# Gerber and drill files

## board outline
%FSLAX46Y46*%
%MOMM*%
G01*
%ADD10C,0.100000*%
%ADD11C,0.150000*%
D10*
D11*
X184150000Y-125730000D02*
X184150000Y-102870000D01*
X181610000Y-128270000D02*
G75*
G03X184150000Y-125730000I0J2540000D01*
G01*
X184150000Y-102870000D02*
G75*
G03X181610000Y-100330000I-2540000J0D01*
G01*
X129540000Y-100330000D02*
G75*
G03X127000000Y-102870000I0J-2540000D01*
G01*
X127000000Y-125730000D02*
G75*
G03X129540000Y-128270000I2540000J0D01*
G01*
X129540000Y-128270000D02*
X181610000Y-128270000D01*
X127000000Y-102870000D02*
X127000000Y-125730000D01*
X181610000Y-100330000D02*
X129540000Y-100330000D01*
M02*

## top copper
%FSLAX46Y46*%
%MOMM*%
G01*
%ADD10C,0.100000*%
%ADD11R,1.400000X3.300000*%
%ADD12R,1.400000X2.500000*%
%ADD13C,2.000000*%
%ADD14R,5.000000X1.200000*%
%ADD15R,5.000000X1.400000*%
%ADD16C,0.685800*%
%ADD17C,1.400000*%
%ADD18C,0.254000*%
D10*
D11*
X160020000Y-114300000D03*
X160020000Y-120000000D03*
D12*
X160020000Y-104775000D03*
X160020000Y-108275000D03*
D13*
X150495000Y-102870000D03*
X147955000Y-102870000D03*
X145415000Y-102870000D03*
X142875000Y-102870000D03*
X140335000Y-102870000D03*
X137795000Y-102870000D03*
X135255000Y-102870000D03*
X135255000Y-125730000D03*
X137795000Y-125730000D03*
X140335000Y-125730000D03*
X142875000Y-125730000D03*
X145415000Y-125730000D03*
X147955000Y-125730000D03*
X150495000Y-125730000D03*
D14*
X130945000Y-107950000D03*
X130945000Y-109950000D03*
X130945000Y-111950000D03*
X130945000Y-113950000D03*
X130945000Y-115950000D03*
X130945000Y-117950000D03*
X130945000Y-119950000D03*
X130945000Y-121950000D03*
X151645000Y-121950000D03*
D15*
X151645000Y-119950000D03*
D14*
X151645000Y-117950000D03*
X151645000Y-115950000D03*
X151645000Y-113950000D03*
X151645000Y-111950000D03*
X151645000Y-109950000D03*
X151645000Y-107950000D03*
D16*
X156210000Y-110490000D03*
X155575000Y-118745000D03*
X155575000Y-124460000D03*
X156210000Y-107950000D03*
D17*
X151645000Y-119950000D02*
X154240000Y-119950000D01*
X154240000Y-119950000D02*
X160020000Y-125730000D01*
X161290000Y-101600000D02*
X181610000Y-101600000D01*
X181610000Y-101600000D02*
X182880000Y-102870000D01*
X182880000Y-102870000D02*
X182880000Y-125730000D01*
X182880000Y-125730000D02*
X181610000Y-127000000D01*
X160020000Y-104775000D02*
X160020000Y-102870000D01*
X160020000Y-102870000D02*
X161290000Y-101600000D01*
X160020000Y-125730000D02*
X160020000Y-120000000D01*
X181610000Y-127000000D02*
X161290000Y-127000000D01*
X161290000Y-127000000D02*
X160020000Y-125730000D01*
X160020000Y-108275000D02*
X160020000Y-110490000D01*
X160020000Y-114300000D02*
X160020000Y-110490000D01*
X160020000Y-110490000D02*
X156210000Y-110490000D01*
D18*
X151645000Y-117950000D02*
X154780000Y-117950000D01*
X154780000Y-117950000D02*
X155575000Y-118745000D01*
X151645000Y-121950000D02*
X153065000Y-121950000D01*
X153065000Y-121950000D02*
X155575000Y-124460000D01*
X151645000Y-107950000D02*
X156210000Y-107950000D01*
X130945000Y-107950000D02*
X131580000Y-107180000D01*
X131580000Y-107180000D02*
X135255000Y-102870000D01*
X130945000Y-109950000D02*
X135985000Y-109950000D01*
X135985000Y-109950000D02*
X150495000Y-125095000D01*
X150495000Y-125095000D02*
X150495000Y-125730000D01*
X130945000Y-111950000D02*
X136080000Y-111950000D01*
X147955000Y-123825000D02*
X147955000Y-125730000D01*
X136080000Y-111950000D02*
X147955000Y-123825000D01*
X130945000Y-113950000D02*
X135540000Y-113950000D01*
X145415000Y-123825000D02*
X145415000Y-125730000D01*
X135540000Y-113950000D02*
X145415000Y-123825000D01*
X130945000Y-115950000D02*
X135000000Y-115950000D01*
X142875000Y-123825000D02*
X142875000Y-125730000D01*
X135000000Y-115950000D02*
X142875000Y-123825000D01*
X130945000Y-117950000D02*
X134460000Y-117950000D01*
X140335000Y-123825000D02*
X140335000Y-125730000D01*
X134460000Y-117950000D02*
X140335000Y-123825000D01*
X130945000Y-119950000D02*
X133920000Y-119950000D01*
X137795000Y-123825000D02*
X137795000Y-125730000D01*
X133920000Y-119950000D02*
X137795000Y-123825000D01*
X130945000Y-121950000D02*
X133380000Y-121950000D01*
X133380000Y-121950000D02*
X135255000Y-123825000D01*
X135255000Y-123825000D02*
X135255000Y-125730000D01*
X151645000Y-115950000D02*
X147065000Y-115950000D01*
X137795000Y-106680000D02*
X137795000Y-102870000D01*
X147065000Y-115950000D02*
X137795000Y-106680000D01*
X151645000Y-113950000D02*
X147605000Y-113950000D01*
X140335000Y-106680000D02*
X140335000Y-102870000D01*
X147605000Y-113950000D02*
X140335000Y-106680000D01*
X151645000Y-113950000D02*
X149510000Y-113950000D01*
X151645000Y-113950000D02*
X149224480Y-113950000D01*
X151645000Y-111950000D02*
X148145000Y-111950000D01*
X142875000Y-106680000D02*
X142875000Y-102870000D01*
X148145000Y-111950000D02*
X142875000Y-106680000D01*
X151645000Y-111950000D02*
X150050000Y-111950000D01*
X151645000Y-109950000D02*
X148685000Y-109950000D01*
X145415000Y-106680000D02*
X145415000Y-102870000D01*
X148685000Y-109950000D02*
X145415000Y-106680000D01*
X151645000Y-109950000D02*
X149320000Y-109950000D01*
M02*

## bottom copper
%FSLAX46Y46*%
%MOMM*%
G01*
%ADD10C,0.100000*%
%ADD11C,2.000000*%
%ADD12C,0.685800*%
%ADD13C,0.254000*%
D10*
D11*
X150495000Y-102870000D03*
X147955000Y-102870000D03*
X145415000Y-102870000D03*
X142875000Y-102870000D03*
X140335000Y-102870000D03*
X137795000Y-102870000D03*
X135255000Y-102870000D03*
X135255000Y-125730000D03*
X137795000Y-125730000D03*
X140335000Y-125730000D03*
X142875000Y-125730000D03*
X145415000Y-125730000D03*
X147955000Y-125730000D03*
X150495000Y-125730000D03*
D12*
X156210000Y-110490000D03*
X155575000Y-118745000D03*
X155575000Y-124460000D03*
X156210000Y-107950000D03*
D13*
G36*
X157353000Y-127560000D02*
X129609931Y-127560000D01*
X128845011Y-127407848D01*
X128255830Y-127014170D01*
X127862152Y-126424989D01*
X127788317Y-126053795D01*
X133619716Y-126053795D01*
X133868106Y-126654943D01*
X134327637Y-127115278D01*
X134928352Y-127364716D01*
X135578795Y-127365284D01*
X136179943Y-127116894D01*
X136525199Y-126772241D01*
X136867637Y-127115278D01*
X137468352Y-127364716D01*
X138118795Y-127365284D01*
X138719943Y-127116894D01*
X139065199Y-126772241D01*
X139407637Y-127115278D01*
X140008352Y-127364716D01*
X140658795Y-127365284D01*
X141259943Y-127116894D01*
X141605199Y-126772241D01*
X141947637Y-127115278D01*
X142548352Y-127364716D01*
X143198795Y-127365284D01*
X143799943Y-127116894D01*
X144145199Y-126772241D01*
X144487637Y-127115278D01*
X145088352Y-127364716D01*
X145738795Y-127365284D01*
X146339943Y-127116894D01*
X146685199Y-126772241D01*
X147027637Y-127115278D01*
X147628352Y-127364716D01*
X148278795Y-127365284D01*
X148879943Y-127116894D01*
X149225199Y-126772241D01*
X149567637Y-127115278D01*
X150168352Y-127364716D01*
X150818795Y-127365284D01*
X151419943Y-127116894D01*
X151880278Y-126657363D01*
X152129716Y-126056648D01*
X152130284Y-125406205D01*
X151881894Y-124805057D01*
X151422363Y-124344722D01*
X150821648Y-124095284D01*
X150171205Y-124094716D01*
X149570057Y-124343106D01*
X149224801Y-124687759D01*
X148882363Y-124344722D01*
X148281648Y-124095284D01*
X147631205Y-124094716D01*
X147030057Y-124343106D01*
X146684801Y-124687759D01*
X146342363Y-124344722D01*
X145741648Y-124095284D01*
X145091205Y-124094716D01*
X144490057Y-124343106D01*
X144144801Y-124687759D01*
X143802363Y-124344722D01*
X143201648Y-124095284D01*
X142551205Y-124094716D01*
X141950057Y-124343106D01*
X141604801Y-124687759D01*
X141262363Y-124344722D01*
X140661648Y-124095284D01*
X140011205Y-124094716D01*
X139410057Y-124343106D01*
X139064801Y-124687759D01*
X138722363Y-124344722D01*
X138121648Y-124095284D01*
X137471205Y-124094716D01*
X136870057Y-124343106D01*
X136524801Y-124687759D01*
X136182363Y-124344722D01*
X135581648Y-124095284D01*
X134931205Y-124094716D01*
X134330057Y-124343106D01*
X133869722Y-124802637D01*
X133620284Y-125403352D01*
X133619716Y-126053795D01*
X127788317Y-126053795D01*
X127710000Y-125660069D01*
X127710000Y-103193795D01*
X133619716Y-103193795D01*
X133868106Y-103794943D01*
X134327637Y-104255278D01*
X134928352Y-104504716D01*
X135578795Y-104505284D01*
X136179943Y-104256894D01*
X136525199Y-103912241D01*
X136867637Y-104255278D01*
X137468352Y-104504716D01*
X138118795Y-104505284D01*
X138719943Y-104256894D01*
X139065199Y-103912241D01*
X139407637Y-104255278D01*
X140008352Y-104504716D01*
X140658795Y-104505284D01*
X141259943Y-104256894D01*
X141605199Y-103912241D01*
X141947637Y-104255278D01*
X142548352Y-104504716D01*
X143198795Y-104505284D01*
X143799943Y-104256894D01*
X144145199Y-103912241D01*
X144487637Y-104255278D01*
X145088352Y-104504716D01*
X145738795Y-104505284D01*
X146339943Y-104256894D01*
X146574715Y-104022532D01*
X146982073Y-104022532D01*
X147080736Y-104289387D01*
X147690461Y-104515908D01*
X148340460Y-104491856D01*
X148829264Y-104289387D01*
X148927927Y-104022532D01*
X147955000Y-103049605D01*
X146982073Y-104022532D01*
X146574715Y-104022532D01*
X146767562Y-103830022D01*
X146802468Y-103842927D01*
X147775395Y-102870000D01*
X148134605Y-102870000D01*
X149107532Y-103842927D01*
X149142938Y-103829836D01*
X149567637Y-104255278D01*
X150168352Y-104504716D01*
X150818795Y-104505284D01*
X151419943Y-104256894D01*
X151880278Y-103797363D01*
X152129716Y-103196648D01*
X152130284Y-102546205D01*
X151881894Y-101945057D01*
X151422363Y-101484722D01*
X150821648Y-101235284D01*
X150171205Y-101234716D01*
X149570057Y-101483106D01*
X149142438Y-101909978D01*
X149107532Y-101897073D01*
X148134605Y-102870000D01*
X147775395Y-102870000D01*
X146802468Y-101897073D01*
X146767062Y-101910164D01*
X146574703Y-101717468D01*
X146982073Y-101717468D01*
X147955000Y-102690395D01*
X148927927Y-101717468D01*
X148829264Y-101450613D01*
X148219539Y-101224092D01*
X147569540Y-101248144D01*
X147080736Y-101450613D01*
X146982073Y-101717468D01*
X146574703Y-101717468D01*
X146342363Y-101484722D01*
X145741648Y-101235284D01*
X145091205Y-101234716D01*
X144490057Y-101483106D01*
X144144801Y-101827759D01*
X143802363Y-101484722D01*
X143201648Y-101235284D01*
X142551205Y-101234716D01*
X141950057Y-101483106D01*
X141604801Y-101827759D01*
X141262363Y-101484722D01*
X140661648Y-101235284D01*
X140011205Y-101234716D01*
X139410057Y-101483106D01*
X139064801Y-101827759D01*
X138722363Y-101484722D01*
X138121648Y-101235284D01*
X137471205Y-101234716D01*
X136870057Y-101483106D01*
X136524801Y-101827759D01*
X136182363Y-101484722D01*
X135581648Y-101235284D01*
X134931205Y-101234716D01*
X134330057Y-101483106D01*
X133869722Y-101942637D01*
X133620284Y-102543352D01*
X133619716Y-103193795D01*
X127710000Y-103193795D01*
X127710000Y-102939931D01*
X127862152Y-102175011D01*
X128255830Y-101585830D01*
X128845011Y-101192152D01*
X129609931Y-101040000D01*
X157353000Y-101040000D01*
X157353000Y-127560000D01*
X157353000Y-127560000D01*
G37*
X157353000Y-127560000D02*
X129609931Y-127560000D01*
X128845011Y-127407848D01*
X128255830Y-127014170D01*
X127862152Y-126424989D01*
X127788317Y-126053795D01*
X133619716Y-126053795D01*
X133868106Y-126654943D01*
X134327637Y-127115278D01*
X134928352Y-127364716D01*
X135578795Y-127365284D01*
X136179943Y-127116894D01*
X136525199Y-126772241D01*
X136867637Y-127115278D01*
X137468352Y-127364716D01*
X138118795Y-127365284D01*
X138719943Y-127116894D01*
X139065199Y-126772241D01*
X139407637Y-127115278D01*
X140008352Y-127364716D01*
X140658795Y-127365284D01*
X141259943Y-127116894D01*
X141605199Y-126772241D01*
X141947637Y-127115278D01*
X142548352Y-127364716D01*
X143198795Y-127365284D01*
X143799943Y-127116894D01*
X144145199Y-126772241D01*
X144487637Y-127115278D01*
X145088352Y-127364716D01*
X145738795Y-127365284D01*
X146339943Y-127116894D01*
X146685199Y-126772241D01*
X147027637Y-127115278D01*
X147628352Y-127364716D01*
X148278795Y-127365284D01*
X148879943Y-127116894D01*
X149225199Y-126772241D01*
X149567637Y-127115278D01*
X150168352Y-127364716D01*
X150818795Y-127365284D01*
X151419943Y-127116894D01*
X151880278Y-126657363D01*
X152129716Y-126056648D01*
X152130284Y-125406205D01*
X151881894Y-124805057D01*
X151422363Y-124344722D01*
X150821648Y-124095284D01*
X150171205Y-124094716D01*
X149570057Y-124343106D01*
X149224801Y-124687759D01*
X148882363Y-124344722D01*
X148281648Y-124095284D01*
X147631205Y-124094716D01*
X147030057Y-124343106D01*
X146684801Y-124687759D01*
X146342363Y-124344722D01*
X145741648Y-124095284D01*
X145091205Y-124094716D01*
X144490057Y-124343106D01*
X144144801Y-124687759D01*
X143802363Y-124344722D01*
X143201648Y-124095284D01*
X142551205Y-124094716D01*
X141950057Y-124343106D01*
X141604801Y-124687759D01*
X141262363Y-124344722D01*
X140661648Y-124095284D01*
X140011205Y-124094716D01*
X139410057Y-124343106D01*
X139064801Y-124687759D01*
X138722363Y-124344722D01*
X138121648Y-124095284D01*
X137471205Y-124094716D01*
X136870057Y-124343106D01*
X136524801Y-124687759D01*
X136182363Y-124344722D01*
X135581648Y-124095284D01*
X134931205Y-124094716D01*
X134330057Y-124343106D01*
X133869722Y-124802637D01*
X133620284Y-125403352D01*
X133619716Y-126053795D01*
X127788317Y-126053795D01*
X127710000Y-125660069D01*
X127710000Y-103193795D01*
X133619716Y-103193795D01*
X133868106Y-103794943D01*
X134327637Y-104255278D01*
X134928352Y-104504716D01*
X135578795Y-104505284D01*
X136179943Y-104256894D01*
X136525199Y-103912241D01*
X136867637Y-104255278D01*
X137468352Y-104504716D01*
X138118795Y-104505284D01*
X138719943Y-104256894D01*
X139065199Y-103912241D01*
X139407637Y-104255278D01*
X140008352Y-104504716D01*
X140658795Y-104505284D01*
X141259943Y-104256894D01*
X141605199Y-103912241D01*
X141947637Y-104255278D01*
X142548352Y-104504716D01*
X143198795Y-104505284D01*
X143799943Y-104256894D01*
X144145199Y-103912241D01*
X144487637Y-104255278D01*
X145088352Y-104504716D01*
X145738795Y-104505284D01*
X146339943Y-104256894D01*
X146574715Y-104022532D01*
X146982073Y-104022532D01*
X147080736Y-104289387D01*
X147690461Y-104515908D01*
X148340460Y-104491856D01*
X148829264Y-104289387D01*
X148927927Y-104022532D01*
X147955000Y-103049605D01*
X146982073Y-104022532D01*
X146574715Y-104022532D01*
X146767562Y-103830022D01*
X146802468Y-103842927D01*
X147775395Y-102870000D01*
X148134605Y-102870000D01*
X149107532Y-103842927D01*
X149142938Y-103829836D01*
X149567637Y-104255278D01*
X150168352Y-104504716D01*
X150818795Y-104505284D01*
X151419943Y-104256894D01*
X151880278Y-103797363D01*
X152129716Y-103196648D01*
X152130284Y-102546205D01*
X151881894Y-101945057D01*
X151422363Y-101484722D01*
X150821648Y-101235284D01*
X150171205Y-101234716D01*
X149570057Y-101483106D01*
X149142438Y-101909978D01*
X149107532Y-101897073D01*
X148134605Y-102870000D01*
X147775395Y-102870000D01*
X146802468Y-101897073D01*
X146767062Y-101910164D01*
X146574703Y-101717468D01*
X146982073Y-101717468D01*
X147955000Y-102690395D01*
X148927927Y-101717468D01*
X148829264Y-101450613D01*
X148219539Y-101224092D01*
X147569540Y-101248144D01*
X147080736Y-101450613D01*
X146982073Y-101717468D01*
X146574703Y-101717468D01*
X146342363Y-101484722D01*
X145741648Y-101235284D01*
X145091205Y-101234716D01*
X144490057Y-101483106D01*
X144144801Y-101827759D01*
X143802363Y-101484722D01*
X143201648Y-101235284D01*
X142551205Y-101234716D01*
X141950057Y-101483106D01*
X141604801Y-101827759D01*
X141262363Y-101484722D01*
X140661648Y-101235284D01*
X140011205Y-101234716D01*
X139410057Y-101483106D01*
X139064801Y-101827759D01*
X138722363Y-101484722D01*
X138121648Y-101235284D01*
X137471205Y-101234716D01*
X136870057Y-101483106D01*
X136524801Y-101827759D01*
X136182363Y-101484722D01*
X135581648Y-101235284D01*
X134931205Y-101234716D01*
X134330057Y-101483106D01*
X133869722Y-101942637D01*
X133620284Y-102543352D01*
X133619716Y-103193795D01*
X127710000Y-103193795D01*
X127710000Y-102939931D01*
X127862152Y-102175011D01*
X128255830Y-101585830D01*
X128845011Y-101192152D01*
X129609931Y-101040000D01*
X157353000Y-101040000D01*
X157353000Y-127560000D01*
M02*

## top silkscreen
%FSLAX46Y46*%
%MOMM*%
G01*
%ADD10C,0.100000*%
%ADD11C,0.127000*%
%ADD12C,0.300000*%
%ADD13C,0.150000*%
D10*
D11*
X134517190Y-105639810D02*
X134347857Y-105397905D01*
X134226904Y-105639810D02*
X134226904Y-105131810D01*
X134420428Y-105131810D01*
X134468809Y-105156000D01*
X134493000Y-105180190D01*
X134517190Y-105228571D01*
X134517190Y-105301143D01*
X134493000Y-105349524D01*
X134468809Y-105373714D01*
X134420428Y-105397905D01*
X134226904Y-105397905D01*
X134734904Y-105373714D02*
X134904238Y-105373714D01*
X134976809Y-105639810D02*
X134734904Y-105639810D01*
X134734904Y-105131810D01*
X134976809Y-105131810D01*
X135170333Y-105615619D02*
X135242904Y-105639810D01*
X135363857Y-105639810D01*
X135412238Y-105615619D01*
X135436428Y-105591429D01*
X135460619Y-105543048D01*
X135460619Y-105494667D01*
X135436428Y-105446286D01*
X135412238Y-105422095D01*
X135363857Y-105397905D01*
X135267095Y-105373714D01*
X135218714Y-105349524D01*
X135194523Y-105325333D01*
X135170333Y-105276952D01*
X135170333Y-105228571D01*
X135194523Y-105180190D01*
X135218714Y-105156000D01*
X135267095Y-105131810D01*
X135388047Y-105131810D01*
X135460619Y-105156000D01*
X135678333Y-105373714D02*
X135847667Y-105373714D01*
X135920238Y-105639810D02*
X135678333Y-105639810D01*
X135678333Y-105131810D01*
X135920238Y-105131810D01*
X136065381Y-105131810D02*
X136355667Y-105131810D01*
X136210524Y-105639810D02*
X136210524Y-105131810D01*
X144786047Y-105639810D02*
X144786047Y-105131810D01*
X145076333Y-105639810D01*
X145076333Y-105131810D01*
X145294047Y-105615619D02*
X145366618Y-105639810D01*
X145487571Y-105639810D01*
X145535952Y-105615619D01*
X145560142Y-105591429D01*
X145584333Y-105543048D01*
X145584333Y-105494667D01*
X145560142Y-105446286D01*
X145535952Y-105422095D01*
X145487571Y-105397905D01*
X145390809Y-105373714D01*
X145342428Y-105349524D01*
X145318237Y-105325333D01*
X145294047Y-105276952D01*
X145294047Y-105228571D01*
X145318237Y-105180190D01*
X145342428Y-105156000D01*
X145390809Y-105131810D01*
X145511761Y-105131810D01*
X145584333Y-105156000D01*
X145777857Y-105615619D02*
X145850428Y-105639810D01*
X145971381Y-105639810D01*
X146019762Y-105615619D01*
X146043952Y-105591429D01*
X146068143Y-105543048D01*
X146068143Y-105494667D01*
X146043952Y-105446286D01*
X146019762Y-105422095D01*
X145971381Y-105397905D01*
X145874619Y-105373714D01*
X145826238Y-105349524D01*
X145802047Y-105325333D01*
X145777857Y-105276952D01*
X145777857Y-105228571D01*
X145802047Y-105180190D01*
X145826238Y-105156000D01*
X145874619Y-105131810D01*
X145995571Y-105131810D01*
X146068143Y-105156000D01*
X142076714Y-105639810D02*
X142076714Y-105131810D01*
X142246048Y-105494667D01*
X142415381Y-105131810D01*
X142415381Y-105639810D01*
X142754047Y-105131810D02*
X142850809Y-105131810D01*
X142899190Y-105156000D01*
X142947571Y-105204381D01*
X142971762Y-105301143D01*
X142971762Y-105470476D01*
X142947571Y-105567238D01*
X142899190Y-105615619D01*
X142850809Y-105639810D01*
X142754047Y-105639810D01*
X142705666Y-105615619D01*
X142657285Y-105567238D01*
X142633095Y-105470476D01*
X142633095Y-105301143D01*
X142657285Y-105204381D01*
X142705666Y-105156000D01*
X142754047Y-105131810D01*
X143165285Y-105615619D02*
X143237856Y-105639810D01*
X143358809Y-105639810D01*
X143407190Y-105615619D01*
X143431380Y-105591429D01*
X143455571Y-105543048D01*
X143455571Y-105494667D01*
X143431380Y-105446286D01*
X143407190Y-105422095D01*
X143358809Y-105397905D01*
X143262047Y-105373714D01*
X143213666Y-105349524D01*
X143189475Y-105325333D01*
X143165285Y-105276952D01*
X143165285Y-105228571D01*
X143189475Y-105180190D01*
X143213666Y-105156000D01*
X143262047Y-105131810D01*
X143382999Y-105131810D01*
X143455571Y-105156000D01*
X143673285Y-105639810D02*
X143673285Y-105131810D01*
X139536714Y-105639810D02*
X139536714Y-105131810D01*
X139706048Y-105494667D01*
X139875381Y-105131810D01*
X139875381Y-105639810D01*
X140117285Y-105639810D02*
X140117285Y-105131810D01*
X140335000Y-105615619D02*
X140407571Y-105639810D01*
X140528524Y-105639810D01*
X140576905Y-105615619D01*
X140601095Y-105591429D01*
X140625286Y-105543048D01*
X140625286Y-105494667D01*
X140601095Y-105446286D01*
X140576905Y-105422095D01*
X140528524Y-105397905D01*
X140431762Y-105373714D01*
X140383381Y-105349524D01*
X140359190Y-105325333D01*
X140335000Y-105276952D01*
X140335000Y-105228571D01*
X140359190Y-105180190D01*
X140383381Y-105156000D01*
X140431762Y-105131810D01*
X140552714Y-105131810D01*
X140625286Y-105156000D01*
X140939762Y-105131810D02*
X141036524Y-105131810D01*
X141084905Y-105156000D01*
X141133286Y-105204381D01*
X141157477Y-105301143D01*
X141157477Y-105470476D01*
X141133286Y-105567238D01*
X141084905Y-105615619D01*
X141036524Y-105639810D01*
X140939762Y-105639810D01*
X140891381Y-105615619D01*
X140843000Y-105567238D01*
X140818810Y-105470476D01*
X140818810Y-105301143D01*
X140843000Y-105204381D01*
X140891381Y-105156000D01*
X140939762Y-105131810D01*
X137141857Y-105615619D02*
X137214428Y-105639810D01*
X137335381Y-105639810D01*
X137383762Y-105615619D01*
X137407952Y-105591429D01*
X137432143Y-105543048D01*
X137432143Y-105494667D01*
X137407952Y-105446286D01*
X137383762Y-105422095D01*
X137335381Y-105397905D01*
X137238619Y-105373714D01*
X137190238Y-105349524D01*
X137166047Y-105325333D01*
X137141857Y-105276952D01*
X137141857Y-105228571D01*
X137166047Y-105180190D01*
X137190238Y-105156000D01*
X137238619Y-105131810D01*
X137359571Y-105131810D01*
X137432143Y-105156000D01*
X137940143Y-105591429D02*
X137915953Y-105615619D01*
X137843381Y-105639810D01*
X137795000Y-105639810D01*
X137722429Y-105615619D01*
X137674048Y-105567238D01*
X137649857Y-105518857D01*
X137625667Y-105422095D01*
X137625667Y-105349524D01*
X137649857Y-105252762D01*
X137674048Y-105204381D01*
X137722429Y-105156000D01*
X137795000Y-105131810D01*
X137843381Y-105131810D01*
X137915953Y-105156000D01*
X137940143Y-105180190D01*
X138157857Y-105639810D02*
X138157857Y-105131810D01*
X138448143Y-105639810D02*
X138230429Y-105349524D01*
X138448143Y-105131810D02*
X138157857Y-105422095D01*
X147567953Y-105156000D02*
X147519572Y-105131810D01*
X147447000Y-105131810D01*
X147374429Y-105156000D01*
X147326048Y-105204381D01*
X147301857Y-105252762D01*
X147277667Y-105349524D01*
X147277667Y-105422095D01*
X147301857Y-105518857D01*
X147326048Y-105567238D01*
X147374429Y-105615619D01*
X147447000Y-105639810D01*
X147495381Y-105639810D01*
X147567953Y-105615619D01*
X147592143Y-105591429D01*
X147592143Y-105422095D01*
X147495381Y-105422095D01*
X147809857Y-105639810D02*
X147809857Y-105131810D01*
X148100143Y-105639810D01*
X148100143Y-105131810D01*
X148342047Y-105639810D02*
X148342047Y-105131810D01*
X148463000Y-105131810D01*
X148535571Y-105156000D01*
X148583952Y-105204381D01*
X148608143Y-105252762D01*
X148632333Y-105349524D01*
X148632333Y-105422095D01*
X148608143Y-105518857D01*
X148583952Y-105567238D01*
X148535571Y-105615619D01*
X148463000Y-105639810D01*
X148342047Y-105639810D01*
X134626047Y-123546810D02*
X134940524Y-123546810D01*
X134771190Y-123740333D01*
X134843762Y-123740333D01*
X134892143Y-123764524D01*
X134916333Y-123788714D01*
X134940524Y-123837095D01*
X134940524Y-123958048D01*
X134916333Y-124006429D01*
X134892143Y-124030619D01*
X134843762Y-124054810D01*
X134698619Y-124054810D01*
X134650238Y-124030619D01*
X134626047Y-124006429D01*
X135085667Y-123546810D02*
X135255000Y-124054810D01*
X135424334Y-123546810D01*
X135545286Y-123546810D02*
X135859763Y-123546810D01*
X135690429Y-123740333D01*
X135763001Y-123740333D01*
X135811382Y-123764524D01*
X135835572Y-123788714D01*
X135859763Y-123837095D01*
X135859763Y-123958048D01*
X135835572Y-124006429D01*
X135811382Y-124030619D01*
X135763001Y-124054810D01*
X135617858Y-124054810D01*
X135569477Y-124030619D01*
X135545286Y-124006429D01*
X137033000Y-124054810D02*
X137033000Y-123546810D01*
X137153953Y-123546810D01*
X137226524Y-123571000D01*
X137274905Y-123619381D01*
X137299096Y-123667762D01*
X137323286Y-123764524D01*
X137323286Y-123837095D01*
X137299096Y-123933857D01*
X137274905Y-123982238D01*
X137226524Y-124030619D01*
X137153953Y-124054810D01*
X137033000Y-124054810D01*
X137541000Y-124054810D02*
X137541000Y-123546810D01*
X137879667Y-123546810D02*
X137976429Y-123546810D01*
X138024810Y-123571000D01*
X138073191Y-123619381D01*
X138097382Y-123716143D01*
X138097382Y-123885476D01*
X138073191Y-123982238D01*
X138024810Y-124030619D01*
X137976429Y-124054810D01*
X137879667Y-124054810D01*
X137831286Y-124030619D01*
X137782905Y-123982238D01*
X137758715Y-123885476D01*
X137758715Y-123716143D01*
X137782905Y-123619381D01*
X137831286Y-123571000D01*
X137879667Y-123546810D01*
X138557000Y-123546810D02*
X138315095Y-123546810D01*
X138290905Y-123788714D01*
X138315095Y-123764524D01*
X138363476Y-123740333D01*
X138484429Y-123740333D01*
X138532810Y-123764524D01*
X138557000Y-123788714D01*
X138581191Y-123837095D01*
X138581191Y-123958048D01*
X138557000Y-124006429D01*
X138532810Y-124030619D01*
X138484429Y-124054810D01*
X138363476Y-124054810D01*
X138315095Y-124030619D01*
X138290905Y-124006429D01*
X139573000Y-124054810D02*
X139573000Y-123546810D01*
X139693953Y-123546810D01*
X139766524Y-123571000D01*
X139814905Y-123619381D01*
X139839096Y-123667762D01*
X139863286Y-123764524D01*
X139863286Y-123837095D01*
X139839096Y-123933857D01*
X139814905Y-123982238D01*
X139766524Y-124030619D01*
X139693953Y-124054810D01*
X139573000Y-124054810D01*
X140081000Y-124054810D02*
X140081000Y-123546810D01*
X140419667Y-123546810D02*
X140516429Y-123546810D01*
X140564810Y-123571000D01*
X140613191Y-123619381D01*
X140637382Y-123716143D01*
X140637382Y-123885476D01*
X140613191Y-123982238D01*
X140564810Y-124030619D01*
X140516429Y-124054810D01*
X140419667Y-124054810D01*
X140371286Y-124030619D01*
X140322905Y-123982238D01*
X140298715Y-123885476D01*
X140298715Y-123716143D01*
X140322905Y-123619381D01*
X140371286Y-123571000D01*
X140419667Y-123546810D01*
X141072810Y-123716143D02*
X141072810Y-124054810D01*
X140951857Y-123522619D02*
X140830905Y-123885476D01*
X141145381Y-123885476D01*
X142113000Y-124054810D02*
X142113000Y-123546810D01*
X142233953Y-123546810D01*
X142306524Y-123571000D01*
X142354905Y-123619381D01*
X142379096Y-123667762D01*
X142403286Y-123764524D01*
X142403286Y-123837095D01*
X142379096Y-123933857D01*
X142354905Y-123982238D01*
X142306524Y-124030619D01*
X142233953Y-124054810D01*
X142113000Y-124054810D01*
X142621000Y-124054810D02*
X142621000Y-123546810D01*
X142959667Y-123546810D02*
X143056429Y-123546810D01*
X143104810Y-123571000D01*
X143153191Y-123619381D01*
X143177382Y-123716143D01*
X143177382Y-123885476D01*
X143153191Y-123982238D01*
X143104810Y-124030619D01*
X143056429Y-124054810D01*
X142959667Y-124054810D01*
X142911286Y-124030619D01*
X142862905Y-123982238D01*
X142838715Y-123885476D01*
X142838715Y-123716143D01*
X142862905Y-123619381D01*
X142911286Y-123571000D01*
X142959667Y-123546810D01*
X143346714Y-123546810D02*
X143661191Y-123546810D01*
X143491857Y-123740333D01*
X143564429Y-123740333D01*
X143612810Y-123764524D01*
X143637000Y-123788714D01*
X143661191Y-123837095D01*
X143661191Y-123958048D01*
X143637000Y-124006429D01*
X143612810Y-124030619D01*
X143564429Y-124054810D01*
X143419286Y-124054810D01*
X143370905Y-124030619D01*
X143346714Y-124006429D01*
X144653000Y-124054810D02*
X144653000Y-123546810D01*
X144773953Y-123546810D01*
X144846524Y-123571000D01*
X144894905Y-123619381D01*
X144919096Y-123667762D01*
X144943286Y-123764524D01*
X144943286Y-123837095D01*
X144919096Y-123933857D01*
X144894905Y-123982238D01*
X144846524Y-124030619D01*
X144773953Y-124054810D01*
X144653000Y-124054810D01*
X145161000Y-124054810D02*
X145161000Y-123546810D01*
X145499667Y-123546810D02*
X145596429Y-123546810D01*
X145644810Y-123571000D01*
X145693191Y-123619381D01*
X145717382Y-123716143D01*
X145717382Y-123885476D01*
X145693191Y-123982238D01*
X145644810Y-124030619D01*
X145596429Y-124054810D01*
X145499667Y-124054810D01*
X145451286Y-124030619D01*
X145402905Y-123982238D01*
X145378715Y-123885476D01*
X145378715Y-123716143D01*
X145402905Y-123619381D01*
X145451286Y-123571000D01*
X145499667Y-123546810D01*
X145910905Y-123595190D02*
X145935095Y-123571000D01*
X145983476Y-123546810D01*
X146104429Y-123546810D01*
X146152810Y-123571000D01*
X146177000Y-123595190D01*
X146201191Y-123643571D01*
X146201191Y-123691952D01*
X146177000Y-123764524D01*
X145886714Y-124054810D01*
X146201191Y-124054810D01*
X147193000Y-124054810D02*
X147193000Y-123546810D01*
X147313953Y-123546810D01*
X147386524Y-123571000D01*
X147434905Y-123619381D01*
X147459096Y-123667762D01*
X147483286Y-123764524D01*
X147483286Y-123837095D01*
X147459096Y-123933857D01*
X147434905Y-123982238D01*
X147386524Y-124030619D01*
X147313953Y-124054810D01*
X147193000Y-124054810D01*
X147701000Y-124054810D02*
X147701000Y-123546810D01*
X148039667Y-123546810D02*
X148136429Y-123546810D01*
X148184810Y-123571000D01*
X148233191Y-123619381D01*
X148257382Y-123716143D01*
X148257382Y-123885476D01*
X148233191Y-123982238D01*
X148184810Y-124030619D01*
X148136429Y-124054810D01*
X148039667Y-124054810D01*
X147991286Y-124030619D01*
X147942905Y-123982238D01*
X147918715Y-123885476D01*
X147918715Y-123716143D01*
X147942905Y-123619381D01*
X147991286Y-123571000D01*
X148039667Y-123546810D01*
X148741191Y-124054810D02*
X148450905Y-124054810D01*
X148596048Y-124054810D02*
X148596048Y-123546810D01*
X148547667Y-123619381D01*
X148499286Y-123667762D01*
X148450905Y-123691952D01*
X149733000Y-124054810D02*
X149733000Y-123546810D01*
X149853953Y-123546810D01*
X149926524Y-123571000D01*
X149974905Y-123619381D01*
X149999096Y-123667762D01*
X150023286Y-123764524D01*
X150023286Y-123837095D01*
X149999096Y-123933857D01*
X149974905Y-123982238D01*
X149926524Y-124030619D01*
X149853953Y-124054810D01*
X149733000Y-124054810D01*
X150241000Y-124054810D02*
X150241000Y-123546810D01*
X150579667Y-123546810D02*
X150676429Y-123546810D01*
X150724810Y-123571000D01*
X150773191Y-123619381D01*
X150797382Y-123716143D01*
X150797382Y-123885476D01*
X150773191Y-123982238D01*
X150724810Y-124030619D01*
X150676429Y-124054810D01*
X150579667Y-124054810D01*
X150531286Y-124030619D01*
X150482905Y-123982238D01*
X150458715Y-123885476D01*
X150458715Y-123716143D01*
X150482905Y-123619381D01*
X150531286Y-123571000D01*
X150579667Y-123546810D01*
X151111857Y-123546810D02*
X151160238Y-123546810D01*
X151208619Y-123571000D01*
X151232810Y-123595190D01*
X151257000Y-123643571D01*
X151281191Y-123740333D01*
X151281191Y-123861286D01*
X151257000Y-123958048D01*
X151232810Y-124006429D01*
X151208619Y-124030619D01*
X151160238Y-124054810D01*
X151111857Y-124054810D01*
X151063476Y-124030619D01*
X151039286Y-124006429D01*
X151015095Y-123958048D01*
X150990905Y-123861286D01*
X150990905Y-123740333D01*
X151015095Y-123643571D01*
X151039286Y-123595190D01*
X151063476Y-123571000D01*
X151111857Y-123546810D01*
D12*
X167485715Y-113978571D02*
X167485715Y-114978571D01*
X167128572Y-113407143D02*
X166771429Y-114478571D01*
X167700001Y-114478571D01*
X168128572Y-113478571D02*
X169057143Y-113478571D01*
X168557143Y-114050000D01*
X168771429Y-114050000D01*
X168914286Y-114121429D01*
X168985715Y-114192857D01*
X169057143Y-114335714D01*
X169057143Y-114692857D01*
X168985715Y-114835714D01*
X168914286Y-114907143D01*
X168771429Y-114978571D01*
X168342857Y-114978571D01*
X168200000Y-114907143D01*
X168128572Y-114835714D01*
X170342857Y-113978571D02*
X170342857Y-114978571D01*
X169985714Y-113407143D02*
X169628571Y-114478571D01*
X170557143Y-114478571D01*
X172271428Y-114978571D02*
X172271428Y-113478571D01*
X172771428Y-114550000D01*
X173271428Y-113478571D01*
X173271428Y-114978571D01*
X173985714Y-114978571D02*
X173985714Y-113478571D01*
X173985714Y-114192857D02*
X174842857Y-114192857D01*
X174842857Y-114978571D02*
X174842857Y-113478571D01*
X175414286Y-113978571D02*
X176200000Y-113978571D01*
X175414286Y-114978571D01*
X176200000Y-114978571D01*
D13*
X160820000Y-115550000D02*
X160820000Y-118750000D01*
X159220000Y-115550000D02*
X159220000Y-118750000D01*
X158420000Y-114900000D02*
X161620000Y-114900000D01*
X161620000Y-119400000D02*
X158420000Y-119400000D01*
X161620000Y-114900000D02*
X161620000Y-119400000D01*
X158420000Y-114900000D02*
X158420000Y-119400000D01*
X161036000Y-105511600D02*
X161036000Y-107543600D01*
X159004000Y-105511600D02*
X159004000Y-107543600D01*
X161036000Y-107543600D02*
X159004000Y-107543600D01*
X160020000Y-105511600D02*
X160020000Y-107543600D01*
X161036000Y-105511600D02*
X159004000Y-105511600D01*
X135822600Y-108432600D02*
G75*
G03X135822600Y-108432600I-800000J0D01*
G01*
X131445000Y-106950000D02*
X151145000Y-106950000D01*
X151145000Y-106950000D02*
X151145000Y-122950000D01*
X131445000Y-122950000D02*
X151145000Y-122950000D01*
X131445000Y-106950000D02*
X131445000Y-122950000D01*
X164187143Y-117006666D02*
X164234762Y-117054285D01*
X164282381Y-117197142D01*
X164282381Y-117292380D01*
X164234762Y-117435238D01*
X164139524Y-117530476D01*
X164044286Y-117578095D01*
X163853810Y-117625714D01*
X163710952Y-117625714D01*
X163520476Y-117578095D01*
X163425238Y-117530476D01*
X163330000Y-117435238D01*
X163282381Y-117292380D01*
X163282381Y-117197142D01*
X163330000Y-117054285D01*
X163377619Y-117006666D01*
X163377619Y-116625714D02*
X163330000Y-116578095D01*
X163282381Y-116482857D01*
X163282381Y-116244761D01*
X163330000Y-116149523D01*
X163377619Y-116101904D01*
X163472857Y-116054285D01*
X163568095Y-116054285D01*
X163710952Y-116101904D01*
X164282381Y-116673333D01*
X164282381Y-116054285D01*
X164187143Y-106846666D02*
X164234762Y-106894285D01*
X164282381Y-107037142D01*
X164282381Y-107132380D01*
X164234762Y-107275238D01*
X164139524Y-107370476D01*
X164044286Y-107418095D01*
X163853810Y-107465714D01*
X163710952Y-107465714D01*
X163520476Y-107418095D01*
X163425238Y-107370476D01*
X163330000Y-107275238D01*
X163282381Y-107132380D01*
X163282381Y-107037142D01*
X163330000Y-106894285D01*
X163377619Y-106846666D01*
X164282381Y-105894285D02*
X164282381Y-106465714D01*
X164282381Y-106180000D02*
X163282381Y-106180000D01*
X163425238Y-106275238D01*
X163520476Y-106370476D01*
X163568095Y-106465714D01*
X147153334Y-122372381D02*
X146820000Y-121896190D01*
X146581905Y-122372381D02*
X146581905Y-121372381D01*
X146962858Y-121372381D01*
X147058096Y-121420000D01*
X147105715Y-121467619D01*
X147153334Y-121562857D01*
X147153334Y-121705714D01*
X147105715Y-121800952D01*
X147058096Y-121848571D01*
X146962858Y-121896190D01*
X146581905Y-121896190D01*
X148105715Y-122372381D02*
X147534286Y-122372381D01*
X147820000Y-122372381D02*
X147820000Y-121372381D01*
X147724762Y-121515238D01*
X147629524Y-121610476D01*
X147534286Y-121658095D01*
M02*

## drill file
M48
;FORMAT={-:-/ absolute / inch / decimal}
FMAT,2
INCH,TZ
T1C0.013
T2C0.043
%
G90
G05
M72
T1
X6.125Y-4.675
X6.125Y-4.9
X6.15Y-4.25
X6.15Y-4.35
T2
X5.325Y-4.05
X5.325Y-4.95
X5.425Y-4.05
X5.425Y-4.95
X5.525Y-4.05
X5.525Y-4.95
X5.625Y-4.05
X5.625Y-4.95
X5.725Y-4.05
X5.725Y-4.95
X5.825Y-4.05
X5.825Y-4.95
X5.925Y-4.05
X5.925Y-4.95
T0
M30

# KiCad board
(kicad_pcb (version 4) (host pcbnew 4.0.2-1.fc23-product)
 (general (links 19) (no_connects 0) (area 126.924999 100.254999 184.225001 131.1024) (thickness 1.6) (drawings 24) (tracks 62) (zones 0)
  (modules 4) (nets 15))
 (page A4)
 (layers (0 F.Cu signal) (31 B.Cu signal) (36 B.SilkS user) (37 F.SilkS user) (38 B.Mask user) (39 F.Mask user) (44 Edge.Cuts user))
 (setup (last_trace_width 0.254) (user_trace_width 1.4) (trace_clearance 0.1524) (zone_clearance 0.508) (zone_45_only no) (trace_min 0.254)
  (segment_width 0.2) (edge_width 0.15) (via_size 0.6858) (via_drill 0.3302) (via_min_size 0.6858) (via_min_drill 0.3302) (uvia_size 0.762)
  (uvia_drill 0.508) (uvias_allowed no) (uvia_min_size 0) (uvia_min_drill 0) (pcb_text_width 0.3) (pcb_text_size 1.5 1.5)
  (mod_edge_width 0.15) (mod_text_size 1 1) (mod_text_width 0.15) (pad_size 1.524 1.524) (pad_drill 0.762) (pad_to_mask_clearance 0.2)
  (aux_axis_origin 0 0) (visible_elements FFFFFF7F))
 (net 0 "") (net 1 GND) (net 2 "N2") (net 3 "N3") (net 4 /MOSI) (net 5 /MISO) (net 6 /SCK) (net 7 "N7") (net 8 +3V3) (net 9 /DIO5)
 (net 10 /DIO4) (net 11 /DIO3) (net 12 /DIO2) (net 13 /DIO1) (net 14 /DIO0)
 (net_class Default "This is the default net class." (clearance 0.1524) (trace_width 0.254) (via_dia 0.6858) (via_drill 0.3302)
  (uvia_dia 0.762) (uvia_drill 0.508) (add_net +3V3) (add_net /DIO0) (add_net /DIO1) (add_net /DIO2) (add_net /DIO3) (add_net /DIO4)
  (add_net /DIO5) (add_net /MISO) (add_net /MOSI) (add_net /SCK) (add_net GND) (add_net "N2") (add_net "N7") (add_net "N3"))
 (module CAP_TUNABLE (layer F.Cu) (at 160.02 114.3 270)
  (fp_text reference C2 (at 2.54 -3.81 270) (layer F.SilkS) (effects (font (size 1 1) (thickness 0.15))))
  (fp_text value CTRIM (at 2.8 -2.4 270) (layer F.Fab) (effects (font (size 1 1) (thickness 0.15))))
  (fp_line (start 1.25 -0.8) (end 4.45 -0.8) (layer F.SilkS) (width 0.15))
  (fp_line (start 1.25 0.8) (end 4.45 0.8) (layer F.SilkS) (width 0.15))
  (fp_line (start 0.6 1.6) (end 0.6 -1.6) (layer F.SilkS) (width 0.15))
  (fp_line (start 5.1 -1.6) (end 5.1 1.6) (layer F.SilkS) (width 0.15))
  (fp_line (start 0.6 -1.6) (end 5.1 -1.6) (layer F.SilkS) (width 0.15))
  (fp_line (start 0.6 1.6) (end 5.1 1.6) (layer F.SilkS) (width 0.15))
  (pad 1 smd rect (at 0 0 270) (size 3.3 1.4) (layers F.Cu F.Mask) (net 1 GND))
  (pad 2 smd rect (at 5.7 0 270) (size 3.3 1.4) (layers F.Cu F.Mask) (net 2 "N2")))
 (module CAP (layer F.Cu) (at 160.02 104.775 270)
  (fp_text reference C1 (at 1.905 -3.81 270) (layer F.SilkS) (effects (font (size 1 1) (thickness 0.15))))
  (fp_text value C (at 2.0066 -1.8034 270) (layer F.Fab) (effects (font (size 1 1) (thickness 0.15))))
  (fp_line (start 0.7366 -1.016) (end 2.7686 -1.016) (layer F.SilkS) (width 0.15))
  (fp_line (start 0.7366 1.016) (end 2.7686 1.016) (layer F.SilkS) (width 0.15))
  (fp_line (start 2.7686 -1.016) (end 2.7686 1.016) (layer F.SilkS) (width 0.15))
  (fp_line (start 0.7366 0) (end 2.7686 0) (layer F.SilkS) (width 0.15))
  (fp_line (start 0.7366 -1.016) (end 0.7366 1.016) (layer F.SilkS) (width 0.15))
  (pad 1 smd rect (at 0 0 270) (size 2.5 1.4) (layers F.Cu F.Mask) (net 2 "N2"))
  (pad 2 smd rect (at 3.5 0 270) (size 2.5 1.4) (layers F.Cu F.Mask) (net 1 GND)))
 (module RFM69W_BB (layer B.Cu) (at 142.875 115.57 180)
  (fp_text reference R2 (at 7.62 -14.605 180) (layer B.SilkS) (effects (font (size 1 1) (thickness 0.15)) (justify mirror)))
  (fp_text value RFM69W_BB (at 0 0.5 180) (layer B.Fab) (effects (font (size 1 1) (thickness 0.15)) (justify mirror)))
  (pad 14 thru_hole circle (at -7.62 12.7 180) (size 2 2) (drill 1.1) (layers *.Cu *.Mask B.SilkS))
  (pad 8 thru_hole circle (at -5.08 12.7 180) (size 2 2) (drill 1.1) (layers *.Cu *.Mask B.SilkS) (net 1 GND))
  (pad 12 thru_hole circle (at -2.54 12.7 180) (size 2 2) (drill 1.1) (layers *.Cu *.Mask B.SilkS) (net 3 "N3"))
  (pad 11 thru_hole circle (at 0 12.7 180) (size 2 2) (drill 1.1) (layers *.Cu *.Mask B.SilkS) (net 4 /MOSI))
  (pad 10 thru_hole circle (at 2.54 12.7 180) (size 2 2) (drill 1.1) (layers *.Cu *.Mask B.SilkS) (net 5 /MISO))
  (pad 9 thru_hole circle (at 5.08 12.7 180) (size 2 2) (drill 1.1) (layers *.Cu *.Mask B.SilkS) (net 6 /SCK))
  (pad 13 thru_hole circle (at 7.62 12.7 180) (size 2 2) (drill 1.1) (layers *.Cu *.Mask B.SilkS) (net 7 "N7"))
  (pad 7 thru_hole circle (at 7.62 -10.16 180) (size 2 2) (drill 1.1) (layers *.Cu *.Mask B.SilkS) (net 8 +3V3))
  (pad 6 thru_hole circle (at 5.08 -10.16 180) (size 2 2) (drill 1.1) (layers *.Cu *.Mask B.SilkS) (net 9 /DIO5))
  (pad 5 thru_hole circle (at 2.54 -10.16 180) (size 2 2) (drill 1.1) (layers *.Cu *.Mask B.SilkS) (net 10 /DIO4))
  (pad 4 thru_hole circle (at 0 -10.16 180) (size 2 2) (drill 1.1) (layers *.Cu *.Mask B.SilkS) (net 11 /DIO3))
  (pad 3 thru_hole circle (at -2.54 -10.16 180) (size 2 2) (drill 1.1) (layers *.Cu *.Mask B.SilkS) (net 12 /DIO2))
  (pad 2 thru_hole circle (at -5.08 -10.16 180) (size 2 2) (drill 1.1) (layers *.Cu *.Mask B.SilkS) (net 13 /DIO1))
  (pad 1 thru_hole circle (at -7.62 -10.16 180) (size 2 2) (drill 1.1) (layers *.Cu *.Mask B.SilkS) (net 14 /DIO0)))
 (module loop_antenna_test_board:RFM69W (layer F.Cu) (at 131.445 107.95)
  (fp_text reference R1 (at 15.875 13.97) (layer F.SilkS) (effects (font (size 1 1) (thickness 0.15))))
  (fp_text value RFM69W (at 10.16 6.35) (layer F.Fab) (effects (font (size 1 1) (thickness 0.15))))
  (fp_circle (center 3.5776 0.4826) (end 3.5776 1.2826) (layer F.SilkS) (width 0.15))
  (fp_line (start 0 -1) (end 19.7 -1) (layer F.SilkS) (width 0.15))
  (fp_line (start 19.7 -1) (end 19.7 15) (layer F.SilkS) (width 0.15))
  (fp_line (start 0 15) (end 19.7 15) (layer F.SilkS) (width 0.15))
  (fp_line (start 0 -1) (end 0 15) (layer F.SilkS) (width 0.15))
  (pad 1 smd rect (at -0.5 0) (size 5 1.2) (layers F.Cu F.Mask) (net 7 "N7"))
  (pad 2 smd rect (at -0.5 2) (size 5 1.2) (layers F.Cu F.Mask) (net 14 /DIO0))
  (pad 3 smd rect (at -0.5 4) (size 5 1.2) (layers F.Cu F.Mask) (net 13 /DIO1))
  (pad 4 smd rect (at -0.5 6) (size 5 1.2) (layers F.Cu F.Mask) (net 12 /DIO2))
  (pad 5 smd rect (at -0.5 8) (size 5 1.2) (layers F.Cu F.Mask) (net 11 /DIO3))
  (pad 6 smd rect (at -0.5 10) (size 5 1.2) (layers F.Cu F.Mask) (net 10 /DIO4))
  (pad 7 smd rect (at -0.5 12) (size 5 1.2) (layers F.Cu F.Mask) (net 9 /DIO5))
  (pad 8 smd rect (at -0.5 14) (size 5 1.2) (layers F.Cu F.Mask) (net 8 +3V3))
  (pad 9 smd rect (at 20.2 14) (size 5 1.2) (layers F.Cu F.Mask) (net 1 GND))
  (pad 10 smd rect (at 20.2 12) (size 5 1.4) (layers F.Cu F.Mask) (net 2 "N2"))
  (pad 11 smd rect (at 20.2 10) (size 5 1.2) (layers F.Cu F.Mask) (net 1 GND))
  (pad 12 smd rect (at 20.2 8) (size 5 1.2) (layers F.Cu F.Mask) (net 6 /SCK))
  (pad 13 smd rect (at 20.2 6) (size 5 1.2) (layers F.Cu F.Mask) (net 5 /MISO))
  (pad 14 smd rect (at 20.2 4) (size 5 1.2) (layers F.Cu F.Mask) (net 4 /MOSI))
  (pad 15 smd rect (at 20.2 2) (size 5 1.2) (layers F.Cu F.Mask) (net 3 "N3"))
  (pad 16 smd rect (at 20.2 0) (size 5 1.2) (layers F.Cu F.Mask) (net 1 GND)))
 (gr_line (start 184.15 125.73) (end 184.15 102.87) (angle 90) (layer Edge.Cuts) (width 0.15))
 (gr_arc (start 181.61 125.73) (end 184.15 125.73) (angle 90) (layer Edge.Cuts) (width 0.15))
 (gr_arc (start 181.61 102.87) (end 181.61 100.33) (angle 90) (layer Edge.Cuts) (width 0.15))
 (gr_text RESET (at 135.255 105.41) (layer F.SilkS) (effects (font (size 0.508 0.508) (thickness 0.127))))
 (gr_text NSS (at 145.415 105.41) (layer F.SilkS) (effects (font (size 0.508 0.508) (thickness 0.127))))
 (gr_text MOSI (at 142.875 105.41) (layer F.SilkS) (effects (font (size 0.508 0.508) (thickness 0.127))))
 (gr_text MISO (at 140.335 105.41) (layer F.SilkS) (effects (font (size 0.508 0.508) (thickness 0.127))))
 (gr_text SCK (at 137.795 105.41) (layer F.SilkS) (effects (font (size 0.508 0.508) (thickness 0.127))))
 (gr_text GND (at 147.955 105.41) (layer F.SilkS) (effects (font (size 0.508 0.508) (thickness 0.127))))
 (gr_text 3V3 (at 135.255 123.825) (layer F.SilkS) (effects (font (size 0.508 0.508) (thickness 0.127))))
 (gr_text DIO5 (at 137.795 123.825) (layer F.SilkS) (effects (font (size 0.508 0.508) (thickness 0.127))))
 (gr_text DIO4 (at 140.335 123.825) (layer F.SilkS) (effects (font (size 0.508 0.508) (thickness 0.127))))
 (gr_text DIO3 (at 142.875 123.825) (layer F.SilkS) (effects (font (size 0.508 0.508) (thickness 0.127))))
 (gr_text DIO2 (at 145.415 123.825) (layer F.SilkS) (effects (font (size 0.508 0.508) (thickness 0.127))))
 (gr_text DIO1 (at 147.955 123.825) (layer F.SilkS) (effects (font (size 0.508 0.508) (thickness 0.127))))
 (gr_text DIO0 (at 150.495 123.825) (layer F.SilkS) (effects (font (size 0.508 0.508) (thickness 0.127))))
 (gr_arc (start 129.54 102.87) (end 127 102.87) (angle 90) (layer Edge.Cuts) (width 0.15))
 (gr_arc (start 129.54 125.73) (end 129.54 128.27) (angle 90) (layer Edge.Cuts) (width 0.15))
 (gr_line (start 129.54 128.27) (end 181.61 128.27) (angle 90) (layer Edge.Cuts) (width 0.15))
 (gr_line (start 127 102.87) (end 127 125.73) (angle 90) (layer Edge.Cuts) (width 0.15))
 (gr_line (start 181.61 100.33) (end 129.54 100.33) (angle 90) (layer Edge.Cuts) (width 0.15))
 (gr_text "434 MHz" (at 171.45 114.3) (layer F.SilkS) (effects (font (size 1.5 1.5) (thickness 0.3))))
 (segment (start 151.645 119.95) (end 154.24 119.95) (width 1.4) (layer F.Cu) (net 2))
 (segment (start 154.24 119.95) (end 160.02 125.73) (width 1.4) (layer F.Cu) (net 2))
 (segment (start 161.29 101.6) (end 181.61 101.6) (width 1.4) (layer F.Cu) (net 2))
 (segment (start 181.61 101.6) (end 182.88 102.87) (width 1.4) (layer F.Cu) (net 2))
 (segment (start 182.88 102.87) (end 182.88 125.73) (width 1.4) (layer F.Cu) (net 2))
 (segment (start 182.88 125.73) (end 181.61 127) (width 1.4) (layer F.Cu) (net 2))
 (segment (start 160.02 104.775) (end 160.02 102.87) (width 1.4) (layer F.Cu) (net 2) (status 10))
 (segment (start 160.02 102.87) (end 161.29 101.6) (width 1.4) (layer F.Cu) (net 2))
 (segment (start 160.02 125.73) (end 160.02 120) (width 1.4) (layer F.Cu) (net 2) (status 20))
 (segment (start 181.61 127) (end 161.29 127) (width 1.4) (layer F.Cu) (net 2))
 (segment (start 161.29 127) (end 160.02 125.73) (width 1.4) (layer F.Cu) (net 2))
 (segment (start 160.02 108.275) (end 160.02 110.49) (width 1.4) (layer F.Cu) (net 1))
 (segment (start 160.02 114.3) (end 160.02 110.49) (width 1.4) (layer F.Cu) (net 1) (status 10))
 (via (at 156.21 110.49) (size 0.6858) (drill 0.3302) (layers F.Cu B.Cu) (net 1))
 (segment (start 160.02 110.49) (end 156.21 110.49) (width 1.4) (layer F.Cu) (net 1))
 (segment (start 151.645 117.95) (end 154.78 117.95) (width 0.254) (layer F.Cu) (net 1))
 (via (at 155.575 118.745) (size 0.6858) (drill 0.3302) (layers F.Cu B.Cu) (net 1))
 (segment (start 154.78 117.95) (end 155.575 118.745) (width 0.254) (layer F.Cu) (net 1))
 (segment (start 151.645 121.95) (end 153.065 121.95) (width 0.254) (layer F.Cu) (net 1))
 (segment (start 153.065 121.95) (end 155.575 124.46) (width 0.254) (layer F.Cu) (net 1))
 (via (at 155.575 124.46) (size 0.6858) (drill 0.3302) (layers F.Cu B.Cu) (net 1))
 (segment (start 151.645 107.95) (end 156.21 107.95) (width 0.254) (layer F.Cu) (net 1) (status 10))
 (via (at 156.21 107.95) (size 0.6858) (drill 0.3302) (layers F.Cu B.Cu) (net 1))
 (segment (start 130.945 107.95) (end 131.58 107.18) (width 0.254) (layer F.Cu) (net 7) (status 10))
 (segment (start 131.58 107.18) (end 135.255 102.87) (width 0.254) (layer F.Cu) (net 7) (status 20))
 (segment (start 130.945 109.95) (end 135.985 109.95) (width 0.254) (layer F.Cu) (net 14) (status 10))
 (segment (start 135.985 109.95) (end 150.495 125.095) (width 0.254) (layer F.Cu) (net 14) (status 20))
 (segment (start 150.495 125.095) (end 150.495 125.73) (width 0.254) (layer F.Cu) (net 14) (status 30))
 (segment (start 130.945 111.95) (end 136.08 111.95) (width 0.254) (layer F.Cu) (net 13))
 (segment (start 147.955 123.825) (end 147.955 125.73) (width 0.254) (layer F.Cu) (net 13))
 (segment (start 136.08 111.95) (end 147.955 123.825) (width 0.254) (layer F.Cu) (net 13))
 (segment (start 130.945 113.95) (end 135.54 113.95) (width 0.254) (layer F.Cu) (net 12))
 (segment (start 145.415 123.825) (end 145.415 125.73) (width 0.254) (layer F.Cu) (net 12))
 (segment (start 135.54 113.95) (end 145.415 123.825) (width 0.254) (layer F.Cu) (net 12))
 (segment (start 130.945 115.95) (end 135 115.95) (width 0.254) (layer F.Cu) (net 11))
 (segment (start 142.875 123.825) (end 142.875 125.73) (width 0.254) (layer F.Cu) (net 11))
 (segment (start 135 115.95) (end 142.875 123.825) (width 0.254) (layer F.Cu) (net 11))
 (segment (start 130.945 117.95) (end 134.46 117.95) (width 0.254) (layer F.Cu) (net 10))
 (segment (start 140.335 123.825) (end 140.335 125.73) (width 0.254) (layer F.Cu) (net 10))
 (segment (start 134.46 117.95) (end 140.335 123.825) (width 0.254) (layer F.Cu) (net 10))
 (segment (start 130.945 119.95) (end 133.92 119.95) (width 0.254) (layer F.Cu) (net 9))
 (segment (start 137.795 123.825) (end 137.795 125.73) (width 0.254) (layer F.Cu) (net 9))
 (segment (start 133.92 119.95) (end 137.795 123.825) (width 0.254) (layer F.Cu) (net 9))
 (segment (start 130.945 121.95) (end 133.38 121.95) (width 0.254) (layer F.Cu) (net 8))
 (segment (start 133.38 121.95) (end 135.255 123.825) (width 0.254) (layer F.Cu) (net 8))
 (segment (start 135.255 123.825) (end 135.255 125.73) (width 0.254) (layer F.Cu) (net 8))
 (segment (start 151.645 115.95) (end 147.065 115.95) (width 0.254) (layer F.Cu) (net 6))
 (segment (start 137.795 106.68) (end 137.795 102.87) (width 0.254) (layer F.Cu) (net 6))
 (segment (start 147.065 115.95) (end 137.795 106.68) (width 0.254) (layer F.Cu) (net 6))
 (segment (start 151.645 113.95) (end 147.605 113.95) (width 0.254) (layer F.Cu) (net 5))
 (segment (start 140.335 106.68) (end 140.335 102.87) (width 0.254) (layer F.Cu) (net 5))
 (segment (start 147.605 113.95) (end 140.335 106.68) (width 0.254) (layer F.Cu) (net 5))
 (segment (start 151.645 113.95) (end 149.51 113.95) (width 0.254) (layer F.Cu) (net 5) (status 30))
 (segment (start 151.645 113.95) (end 149.22448 113.95) (width 0.254) (layer F.Cu) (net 5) (status 30))
 (segment (start 151.645 111.95) (end 148.145 111.95) (width 0.254) (layer F.Cu) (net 4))
 (segment (start 142.875 106.68) (end 142.875 102.87) (width 0.254) (layer F.Cu) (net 4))
 (segment (start 148.145 111.95) (end 142.875 106.68) (width 0.254) (layer F.Cu) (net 4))
 (segment (start 151.645 111.95) (end 150.05 111.95) (width 0.254) (layer F.Cu) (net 4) (status 30))
 (segment (start 151.645 109.95) (end 148.685 109.95) (width 0.254) (layer F.Cu) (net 3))
 (segment (start 145.415 106.68) (end 145.415 102.87) (width 0.254) (layer F.Cu) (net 3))
 (segment (start 148.685 109.95) (end 145.415 106.68) (width 0.254) (layer F.Cu) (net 3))
 (segment (start 151.645 109.95) (end 149.32 109.95) (width 0.254) (layer F.Cu) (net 3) (status 10))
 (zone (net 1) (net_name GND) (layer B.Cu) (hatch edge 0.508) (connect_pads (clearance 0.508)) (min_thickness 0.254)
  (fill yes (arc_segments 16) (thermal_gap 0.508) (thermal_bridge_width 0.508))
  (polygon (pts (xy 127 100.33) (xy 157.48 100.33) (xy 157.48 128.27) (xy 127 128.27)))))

